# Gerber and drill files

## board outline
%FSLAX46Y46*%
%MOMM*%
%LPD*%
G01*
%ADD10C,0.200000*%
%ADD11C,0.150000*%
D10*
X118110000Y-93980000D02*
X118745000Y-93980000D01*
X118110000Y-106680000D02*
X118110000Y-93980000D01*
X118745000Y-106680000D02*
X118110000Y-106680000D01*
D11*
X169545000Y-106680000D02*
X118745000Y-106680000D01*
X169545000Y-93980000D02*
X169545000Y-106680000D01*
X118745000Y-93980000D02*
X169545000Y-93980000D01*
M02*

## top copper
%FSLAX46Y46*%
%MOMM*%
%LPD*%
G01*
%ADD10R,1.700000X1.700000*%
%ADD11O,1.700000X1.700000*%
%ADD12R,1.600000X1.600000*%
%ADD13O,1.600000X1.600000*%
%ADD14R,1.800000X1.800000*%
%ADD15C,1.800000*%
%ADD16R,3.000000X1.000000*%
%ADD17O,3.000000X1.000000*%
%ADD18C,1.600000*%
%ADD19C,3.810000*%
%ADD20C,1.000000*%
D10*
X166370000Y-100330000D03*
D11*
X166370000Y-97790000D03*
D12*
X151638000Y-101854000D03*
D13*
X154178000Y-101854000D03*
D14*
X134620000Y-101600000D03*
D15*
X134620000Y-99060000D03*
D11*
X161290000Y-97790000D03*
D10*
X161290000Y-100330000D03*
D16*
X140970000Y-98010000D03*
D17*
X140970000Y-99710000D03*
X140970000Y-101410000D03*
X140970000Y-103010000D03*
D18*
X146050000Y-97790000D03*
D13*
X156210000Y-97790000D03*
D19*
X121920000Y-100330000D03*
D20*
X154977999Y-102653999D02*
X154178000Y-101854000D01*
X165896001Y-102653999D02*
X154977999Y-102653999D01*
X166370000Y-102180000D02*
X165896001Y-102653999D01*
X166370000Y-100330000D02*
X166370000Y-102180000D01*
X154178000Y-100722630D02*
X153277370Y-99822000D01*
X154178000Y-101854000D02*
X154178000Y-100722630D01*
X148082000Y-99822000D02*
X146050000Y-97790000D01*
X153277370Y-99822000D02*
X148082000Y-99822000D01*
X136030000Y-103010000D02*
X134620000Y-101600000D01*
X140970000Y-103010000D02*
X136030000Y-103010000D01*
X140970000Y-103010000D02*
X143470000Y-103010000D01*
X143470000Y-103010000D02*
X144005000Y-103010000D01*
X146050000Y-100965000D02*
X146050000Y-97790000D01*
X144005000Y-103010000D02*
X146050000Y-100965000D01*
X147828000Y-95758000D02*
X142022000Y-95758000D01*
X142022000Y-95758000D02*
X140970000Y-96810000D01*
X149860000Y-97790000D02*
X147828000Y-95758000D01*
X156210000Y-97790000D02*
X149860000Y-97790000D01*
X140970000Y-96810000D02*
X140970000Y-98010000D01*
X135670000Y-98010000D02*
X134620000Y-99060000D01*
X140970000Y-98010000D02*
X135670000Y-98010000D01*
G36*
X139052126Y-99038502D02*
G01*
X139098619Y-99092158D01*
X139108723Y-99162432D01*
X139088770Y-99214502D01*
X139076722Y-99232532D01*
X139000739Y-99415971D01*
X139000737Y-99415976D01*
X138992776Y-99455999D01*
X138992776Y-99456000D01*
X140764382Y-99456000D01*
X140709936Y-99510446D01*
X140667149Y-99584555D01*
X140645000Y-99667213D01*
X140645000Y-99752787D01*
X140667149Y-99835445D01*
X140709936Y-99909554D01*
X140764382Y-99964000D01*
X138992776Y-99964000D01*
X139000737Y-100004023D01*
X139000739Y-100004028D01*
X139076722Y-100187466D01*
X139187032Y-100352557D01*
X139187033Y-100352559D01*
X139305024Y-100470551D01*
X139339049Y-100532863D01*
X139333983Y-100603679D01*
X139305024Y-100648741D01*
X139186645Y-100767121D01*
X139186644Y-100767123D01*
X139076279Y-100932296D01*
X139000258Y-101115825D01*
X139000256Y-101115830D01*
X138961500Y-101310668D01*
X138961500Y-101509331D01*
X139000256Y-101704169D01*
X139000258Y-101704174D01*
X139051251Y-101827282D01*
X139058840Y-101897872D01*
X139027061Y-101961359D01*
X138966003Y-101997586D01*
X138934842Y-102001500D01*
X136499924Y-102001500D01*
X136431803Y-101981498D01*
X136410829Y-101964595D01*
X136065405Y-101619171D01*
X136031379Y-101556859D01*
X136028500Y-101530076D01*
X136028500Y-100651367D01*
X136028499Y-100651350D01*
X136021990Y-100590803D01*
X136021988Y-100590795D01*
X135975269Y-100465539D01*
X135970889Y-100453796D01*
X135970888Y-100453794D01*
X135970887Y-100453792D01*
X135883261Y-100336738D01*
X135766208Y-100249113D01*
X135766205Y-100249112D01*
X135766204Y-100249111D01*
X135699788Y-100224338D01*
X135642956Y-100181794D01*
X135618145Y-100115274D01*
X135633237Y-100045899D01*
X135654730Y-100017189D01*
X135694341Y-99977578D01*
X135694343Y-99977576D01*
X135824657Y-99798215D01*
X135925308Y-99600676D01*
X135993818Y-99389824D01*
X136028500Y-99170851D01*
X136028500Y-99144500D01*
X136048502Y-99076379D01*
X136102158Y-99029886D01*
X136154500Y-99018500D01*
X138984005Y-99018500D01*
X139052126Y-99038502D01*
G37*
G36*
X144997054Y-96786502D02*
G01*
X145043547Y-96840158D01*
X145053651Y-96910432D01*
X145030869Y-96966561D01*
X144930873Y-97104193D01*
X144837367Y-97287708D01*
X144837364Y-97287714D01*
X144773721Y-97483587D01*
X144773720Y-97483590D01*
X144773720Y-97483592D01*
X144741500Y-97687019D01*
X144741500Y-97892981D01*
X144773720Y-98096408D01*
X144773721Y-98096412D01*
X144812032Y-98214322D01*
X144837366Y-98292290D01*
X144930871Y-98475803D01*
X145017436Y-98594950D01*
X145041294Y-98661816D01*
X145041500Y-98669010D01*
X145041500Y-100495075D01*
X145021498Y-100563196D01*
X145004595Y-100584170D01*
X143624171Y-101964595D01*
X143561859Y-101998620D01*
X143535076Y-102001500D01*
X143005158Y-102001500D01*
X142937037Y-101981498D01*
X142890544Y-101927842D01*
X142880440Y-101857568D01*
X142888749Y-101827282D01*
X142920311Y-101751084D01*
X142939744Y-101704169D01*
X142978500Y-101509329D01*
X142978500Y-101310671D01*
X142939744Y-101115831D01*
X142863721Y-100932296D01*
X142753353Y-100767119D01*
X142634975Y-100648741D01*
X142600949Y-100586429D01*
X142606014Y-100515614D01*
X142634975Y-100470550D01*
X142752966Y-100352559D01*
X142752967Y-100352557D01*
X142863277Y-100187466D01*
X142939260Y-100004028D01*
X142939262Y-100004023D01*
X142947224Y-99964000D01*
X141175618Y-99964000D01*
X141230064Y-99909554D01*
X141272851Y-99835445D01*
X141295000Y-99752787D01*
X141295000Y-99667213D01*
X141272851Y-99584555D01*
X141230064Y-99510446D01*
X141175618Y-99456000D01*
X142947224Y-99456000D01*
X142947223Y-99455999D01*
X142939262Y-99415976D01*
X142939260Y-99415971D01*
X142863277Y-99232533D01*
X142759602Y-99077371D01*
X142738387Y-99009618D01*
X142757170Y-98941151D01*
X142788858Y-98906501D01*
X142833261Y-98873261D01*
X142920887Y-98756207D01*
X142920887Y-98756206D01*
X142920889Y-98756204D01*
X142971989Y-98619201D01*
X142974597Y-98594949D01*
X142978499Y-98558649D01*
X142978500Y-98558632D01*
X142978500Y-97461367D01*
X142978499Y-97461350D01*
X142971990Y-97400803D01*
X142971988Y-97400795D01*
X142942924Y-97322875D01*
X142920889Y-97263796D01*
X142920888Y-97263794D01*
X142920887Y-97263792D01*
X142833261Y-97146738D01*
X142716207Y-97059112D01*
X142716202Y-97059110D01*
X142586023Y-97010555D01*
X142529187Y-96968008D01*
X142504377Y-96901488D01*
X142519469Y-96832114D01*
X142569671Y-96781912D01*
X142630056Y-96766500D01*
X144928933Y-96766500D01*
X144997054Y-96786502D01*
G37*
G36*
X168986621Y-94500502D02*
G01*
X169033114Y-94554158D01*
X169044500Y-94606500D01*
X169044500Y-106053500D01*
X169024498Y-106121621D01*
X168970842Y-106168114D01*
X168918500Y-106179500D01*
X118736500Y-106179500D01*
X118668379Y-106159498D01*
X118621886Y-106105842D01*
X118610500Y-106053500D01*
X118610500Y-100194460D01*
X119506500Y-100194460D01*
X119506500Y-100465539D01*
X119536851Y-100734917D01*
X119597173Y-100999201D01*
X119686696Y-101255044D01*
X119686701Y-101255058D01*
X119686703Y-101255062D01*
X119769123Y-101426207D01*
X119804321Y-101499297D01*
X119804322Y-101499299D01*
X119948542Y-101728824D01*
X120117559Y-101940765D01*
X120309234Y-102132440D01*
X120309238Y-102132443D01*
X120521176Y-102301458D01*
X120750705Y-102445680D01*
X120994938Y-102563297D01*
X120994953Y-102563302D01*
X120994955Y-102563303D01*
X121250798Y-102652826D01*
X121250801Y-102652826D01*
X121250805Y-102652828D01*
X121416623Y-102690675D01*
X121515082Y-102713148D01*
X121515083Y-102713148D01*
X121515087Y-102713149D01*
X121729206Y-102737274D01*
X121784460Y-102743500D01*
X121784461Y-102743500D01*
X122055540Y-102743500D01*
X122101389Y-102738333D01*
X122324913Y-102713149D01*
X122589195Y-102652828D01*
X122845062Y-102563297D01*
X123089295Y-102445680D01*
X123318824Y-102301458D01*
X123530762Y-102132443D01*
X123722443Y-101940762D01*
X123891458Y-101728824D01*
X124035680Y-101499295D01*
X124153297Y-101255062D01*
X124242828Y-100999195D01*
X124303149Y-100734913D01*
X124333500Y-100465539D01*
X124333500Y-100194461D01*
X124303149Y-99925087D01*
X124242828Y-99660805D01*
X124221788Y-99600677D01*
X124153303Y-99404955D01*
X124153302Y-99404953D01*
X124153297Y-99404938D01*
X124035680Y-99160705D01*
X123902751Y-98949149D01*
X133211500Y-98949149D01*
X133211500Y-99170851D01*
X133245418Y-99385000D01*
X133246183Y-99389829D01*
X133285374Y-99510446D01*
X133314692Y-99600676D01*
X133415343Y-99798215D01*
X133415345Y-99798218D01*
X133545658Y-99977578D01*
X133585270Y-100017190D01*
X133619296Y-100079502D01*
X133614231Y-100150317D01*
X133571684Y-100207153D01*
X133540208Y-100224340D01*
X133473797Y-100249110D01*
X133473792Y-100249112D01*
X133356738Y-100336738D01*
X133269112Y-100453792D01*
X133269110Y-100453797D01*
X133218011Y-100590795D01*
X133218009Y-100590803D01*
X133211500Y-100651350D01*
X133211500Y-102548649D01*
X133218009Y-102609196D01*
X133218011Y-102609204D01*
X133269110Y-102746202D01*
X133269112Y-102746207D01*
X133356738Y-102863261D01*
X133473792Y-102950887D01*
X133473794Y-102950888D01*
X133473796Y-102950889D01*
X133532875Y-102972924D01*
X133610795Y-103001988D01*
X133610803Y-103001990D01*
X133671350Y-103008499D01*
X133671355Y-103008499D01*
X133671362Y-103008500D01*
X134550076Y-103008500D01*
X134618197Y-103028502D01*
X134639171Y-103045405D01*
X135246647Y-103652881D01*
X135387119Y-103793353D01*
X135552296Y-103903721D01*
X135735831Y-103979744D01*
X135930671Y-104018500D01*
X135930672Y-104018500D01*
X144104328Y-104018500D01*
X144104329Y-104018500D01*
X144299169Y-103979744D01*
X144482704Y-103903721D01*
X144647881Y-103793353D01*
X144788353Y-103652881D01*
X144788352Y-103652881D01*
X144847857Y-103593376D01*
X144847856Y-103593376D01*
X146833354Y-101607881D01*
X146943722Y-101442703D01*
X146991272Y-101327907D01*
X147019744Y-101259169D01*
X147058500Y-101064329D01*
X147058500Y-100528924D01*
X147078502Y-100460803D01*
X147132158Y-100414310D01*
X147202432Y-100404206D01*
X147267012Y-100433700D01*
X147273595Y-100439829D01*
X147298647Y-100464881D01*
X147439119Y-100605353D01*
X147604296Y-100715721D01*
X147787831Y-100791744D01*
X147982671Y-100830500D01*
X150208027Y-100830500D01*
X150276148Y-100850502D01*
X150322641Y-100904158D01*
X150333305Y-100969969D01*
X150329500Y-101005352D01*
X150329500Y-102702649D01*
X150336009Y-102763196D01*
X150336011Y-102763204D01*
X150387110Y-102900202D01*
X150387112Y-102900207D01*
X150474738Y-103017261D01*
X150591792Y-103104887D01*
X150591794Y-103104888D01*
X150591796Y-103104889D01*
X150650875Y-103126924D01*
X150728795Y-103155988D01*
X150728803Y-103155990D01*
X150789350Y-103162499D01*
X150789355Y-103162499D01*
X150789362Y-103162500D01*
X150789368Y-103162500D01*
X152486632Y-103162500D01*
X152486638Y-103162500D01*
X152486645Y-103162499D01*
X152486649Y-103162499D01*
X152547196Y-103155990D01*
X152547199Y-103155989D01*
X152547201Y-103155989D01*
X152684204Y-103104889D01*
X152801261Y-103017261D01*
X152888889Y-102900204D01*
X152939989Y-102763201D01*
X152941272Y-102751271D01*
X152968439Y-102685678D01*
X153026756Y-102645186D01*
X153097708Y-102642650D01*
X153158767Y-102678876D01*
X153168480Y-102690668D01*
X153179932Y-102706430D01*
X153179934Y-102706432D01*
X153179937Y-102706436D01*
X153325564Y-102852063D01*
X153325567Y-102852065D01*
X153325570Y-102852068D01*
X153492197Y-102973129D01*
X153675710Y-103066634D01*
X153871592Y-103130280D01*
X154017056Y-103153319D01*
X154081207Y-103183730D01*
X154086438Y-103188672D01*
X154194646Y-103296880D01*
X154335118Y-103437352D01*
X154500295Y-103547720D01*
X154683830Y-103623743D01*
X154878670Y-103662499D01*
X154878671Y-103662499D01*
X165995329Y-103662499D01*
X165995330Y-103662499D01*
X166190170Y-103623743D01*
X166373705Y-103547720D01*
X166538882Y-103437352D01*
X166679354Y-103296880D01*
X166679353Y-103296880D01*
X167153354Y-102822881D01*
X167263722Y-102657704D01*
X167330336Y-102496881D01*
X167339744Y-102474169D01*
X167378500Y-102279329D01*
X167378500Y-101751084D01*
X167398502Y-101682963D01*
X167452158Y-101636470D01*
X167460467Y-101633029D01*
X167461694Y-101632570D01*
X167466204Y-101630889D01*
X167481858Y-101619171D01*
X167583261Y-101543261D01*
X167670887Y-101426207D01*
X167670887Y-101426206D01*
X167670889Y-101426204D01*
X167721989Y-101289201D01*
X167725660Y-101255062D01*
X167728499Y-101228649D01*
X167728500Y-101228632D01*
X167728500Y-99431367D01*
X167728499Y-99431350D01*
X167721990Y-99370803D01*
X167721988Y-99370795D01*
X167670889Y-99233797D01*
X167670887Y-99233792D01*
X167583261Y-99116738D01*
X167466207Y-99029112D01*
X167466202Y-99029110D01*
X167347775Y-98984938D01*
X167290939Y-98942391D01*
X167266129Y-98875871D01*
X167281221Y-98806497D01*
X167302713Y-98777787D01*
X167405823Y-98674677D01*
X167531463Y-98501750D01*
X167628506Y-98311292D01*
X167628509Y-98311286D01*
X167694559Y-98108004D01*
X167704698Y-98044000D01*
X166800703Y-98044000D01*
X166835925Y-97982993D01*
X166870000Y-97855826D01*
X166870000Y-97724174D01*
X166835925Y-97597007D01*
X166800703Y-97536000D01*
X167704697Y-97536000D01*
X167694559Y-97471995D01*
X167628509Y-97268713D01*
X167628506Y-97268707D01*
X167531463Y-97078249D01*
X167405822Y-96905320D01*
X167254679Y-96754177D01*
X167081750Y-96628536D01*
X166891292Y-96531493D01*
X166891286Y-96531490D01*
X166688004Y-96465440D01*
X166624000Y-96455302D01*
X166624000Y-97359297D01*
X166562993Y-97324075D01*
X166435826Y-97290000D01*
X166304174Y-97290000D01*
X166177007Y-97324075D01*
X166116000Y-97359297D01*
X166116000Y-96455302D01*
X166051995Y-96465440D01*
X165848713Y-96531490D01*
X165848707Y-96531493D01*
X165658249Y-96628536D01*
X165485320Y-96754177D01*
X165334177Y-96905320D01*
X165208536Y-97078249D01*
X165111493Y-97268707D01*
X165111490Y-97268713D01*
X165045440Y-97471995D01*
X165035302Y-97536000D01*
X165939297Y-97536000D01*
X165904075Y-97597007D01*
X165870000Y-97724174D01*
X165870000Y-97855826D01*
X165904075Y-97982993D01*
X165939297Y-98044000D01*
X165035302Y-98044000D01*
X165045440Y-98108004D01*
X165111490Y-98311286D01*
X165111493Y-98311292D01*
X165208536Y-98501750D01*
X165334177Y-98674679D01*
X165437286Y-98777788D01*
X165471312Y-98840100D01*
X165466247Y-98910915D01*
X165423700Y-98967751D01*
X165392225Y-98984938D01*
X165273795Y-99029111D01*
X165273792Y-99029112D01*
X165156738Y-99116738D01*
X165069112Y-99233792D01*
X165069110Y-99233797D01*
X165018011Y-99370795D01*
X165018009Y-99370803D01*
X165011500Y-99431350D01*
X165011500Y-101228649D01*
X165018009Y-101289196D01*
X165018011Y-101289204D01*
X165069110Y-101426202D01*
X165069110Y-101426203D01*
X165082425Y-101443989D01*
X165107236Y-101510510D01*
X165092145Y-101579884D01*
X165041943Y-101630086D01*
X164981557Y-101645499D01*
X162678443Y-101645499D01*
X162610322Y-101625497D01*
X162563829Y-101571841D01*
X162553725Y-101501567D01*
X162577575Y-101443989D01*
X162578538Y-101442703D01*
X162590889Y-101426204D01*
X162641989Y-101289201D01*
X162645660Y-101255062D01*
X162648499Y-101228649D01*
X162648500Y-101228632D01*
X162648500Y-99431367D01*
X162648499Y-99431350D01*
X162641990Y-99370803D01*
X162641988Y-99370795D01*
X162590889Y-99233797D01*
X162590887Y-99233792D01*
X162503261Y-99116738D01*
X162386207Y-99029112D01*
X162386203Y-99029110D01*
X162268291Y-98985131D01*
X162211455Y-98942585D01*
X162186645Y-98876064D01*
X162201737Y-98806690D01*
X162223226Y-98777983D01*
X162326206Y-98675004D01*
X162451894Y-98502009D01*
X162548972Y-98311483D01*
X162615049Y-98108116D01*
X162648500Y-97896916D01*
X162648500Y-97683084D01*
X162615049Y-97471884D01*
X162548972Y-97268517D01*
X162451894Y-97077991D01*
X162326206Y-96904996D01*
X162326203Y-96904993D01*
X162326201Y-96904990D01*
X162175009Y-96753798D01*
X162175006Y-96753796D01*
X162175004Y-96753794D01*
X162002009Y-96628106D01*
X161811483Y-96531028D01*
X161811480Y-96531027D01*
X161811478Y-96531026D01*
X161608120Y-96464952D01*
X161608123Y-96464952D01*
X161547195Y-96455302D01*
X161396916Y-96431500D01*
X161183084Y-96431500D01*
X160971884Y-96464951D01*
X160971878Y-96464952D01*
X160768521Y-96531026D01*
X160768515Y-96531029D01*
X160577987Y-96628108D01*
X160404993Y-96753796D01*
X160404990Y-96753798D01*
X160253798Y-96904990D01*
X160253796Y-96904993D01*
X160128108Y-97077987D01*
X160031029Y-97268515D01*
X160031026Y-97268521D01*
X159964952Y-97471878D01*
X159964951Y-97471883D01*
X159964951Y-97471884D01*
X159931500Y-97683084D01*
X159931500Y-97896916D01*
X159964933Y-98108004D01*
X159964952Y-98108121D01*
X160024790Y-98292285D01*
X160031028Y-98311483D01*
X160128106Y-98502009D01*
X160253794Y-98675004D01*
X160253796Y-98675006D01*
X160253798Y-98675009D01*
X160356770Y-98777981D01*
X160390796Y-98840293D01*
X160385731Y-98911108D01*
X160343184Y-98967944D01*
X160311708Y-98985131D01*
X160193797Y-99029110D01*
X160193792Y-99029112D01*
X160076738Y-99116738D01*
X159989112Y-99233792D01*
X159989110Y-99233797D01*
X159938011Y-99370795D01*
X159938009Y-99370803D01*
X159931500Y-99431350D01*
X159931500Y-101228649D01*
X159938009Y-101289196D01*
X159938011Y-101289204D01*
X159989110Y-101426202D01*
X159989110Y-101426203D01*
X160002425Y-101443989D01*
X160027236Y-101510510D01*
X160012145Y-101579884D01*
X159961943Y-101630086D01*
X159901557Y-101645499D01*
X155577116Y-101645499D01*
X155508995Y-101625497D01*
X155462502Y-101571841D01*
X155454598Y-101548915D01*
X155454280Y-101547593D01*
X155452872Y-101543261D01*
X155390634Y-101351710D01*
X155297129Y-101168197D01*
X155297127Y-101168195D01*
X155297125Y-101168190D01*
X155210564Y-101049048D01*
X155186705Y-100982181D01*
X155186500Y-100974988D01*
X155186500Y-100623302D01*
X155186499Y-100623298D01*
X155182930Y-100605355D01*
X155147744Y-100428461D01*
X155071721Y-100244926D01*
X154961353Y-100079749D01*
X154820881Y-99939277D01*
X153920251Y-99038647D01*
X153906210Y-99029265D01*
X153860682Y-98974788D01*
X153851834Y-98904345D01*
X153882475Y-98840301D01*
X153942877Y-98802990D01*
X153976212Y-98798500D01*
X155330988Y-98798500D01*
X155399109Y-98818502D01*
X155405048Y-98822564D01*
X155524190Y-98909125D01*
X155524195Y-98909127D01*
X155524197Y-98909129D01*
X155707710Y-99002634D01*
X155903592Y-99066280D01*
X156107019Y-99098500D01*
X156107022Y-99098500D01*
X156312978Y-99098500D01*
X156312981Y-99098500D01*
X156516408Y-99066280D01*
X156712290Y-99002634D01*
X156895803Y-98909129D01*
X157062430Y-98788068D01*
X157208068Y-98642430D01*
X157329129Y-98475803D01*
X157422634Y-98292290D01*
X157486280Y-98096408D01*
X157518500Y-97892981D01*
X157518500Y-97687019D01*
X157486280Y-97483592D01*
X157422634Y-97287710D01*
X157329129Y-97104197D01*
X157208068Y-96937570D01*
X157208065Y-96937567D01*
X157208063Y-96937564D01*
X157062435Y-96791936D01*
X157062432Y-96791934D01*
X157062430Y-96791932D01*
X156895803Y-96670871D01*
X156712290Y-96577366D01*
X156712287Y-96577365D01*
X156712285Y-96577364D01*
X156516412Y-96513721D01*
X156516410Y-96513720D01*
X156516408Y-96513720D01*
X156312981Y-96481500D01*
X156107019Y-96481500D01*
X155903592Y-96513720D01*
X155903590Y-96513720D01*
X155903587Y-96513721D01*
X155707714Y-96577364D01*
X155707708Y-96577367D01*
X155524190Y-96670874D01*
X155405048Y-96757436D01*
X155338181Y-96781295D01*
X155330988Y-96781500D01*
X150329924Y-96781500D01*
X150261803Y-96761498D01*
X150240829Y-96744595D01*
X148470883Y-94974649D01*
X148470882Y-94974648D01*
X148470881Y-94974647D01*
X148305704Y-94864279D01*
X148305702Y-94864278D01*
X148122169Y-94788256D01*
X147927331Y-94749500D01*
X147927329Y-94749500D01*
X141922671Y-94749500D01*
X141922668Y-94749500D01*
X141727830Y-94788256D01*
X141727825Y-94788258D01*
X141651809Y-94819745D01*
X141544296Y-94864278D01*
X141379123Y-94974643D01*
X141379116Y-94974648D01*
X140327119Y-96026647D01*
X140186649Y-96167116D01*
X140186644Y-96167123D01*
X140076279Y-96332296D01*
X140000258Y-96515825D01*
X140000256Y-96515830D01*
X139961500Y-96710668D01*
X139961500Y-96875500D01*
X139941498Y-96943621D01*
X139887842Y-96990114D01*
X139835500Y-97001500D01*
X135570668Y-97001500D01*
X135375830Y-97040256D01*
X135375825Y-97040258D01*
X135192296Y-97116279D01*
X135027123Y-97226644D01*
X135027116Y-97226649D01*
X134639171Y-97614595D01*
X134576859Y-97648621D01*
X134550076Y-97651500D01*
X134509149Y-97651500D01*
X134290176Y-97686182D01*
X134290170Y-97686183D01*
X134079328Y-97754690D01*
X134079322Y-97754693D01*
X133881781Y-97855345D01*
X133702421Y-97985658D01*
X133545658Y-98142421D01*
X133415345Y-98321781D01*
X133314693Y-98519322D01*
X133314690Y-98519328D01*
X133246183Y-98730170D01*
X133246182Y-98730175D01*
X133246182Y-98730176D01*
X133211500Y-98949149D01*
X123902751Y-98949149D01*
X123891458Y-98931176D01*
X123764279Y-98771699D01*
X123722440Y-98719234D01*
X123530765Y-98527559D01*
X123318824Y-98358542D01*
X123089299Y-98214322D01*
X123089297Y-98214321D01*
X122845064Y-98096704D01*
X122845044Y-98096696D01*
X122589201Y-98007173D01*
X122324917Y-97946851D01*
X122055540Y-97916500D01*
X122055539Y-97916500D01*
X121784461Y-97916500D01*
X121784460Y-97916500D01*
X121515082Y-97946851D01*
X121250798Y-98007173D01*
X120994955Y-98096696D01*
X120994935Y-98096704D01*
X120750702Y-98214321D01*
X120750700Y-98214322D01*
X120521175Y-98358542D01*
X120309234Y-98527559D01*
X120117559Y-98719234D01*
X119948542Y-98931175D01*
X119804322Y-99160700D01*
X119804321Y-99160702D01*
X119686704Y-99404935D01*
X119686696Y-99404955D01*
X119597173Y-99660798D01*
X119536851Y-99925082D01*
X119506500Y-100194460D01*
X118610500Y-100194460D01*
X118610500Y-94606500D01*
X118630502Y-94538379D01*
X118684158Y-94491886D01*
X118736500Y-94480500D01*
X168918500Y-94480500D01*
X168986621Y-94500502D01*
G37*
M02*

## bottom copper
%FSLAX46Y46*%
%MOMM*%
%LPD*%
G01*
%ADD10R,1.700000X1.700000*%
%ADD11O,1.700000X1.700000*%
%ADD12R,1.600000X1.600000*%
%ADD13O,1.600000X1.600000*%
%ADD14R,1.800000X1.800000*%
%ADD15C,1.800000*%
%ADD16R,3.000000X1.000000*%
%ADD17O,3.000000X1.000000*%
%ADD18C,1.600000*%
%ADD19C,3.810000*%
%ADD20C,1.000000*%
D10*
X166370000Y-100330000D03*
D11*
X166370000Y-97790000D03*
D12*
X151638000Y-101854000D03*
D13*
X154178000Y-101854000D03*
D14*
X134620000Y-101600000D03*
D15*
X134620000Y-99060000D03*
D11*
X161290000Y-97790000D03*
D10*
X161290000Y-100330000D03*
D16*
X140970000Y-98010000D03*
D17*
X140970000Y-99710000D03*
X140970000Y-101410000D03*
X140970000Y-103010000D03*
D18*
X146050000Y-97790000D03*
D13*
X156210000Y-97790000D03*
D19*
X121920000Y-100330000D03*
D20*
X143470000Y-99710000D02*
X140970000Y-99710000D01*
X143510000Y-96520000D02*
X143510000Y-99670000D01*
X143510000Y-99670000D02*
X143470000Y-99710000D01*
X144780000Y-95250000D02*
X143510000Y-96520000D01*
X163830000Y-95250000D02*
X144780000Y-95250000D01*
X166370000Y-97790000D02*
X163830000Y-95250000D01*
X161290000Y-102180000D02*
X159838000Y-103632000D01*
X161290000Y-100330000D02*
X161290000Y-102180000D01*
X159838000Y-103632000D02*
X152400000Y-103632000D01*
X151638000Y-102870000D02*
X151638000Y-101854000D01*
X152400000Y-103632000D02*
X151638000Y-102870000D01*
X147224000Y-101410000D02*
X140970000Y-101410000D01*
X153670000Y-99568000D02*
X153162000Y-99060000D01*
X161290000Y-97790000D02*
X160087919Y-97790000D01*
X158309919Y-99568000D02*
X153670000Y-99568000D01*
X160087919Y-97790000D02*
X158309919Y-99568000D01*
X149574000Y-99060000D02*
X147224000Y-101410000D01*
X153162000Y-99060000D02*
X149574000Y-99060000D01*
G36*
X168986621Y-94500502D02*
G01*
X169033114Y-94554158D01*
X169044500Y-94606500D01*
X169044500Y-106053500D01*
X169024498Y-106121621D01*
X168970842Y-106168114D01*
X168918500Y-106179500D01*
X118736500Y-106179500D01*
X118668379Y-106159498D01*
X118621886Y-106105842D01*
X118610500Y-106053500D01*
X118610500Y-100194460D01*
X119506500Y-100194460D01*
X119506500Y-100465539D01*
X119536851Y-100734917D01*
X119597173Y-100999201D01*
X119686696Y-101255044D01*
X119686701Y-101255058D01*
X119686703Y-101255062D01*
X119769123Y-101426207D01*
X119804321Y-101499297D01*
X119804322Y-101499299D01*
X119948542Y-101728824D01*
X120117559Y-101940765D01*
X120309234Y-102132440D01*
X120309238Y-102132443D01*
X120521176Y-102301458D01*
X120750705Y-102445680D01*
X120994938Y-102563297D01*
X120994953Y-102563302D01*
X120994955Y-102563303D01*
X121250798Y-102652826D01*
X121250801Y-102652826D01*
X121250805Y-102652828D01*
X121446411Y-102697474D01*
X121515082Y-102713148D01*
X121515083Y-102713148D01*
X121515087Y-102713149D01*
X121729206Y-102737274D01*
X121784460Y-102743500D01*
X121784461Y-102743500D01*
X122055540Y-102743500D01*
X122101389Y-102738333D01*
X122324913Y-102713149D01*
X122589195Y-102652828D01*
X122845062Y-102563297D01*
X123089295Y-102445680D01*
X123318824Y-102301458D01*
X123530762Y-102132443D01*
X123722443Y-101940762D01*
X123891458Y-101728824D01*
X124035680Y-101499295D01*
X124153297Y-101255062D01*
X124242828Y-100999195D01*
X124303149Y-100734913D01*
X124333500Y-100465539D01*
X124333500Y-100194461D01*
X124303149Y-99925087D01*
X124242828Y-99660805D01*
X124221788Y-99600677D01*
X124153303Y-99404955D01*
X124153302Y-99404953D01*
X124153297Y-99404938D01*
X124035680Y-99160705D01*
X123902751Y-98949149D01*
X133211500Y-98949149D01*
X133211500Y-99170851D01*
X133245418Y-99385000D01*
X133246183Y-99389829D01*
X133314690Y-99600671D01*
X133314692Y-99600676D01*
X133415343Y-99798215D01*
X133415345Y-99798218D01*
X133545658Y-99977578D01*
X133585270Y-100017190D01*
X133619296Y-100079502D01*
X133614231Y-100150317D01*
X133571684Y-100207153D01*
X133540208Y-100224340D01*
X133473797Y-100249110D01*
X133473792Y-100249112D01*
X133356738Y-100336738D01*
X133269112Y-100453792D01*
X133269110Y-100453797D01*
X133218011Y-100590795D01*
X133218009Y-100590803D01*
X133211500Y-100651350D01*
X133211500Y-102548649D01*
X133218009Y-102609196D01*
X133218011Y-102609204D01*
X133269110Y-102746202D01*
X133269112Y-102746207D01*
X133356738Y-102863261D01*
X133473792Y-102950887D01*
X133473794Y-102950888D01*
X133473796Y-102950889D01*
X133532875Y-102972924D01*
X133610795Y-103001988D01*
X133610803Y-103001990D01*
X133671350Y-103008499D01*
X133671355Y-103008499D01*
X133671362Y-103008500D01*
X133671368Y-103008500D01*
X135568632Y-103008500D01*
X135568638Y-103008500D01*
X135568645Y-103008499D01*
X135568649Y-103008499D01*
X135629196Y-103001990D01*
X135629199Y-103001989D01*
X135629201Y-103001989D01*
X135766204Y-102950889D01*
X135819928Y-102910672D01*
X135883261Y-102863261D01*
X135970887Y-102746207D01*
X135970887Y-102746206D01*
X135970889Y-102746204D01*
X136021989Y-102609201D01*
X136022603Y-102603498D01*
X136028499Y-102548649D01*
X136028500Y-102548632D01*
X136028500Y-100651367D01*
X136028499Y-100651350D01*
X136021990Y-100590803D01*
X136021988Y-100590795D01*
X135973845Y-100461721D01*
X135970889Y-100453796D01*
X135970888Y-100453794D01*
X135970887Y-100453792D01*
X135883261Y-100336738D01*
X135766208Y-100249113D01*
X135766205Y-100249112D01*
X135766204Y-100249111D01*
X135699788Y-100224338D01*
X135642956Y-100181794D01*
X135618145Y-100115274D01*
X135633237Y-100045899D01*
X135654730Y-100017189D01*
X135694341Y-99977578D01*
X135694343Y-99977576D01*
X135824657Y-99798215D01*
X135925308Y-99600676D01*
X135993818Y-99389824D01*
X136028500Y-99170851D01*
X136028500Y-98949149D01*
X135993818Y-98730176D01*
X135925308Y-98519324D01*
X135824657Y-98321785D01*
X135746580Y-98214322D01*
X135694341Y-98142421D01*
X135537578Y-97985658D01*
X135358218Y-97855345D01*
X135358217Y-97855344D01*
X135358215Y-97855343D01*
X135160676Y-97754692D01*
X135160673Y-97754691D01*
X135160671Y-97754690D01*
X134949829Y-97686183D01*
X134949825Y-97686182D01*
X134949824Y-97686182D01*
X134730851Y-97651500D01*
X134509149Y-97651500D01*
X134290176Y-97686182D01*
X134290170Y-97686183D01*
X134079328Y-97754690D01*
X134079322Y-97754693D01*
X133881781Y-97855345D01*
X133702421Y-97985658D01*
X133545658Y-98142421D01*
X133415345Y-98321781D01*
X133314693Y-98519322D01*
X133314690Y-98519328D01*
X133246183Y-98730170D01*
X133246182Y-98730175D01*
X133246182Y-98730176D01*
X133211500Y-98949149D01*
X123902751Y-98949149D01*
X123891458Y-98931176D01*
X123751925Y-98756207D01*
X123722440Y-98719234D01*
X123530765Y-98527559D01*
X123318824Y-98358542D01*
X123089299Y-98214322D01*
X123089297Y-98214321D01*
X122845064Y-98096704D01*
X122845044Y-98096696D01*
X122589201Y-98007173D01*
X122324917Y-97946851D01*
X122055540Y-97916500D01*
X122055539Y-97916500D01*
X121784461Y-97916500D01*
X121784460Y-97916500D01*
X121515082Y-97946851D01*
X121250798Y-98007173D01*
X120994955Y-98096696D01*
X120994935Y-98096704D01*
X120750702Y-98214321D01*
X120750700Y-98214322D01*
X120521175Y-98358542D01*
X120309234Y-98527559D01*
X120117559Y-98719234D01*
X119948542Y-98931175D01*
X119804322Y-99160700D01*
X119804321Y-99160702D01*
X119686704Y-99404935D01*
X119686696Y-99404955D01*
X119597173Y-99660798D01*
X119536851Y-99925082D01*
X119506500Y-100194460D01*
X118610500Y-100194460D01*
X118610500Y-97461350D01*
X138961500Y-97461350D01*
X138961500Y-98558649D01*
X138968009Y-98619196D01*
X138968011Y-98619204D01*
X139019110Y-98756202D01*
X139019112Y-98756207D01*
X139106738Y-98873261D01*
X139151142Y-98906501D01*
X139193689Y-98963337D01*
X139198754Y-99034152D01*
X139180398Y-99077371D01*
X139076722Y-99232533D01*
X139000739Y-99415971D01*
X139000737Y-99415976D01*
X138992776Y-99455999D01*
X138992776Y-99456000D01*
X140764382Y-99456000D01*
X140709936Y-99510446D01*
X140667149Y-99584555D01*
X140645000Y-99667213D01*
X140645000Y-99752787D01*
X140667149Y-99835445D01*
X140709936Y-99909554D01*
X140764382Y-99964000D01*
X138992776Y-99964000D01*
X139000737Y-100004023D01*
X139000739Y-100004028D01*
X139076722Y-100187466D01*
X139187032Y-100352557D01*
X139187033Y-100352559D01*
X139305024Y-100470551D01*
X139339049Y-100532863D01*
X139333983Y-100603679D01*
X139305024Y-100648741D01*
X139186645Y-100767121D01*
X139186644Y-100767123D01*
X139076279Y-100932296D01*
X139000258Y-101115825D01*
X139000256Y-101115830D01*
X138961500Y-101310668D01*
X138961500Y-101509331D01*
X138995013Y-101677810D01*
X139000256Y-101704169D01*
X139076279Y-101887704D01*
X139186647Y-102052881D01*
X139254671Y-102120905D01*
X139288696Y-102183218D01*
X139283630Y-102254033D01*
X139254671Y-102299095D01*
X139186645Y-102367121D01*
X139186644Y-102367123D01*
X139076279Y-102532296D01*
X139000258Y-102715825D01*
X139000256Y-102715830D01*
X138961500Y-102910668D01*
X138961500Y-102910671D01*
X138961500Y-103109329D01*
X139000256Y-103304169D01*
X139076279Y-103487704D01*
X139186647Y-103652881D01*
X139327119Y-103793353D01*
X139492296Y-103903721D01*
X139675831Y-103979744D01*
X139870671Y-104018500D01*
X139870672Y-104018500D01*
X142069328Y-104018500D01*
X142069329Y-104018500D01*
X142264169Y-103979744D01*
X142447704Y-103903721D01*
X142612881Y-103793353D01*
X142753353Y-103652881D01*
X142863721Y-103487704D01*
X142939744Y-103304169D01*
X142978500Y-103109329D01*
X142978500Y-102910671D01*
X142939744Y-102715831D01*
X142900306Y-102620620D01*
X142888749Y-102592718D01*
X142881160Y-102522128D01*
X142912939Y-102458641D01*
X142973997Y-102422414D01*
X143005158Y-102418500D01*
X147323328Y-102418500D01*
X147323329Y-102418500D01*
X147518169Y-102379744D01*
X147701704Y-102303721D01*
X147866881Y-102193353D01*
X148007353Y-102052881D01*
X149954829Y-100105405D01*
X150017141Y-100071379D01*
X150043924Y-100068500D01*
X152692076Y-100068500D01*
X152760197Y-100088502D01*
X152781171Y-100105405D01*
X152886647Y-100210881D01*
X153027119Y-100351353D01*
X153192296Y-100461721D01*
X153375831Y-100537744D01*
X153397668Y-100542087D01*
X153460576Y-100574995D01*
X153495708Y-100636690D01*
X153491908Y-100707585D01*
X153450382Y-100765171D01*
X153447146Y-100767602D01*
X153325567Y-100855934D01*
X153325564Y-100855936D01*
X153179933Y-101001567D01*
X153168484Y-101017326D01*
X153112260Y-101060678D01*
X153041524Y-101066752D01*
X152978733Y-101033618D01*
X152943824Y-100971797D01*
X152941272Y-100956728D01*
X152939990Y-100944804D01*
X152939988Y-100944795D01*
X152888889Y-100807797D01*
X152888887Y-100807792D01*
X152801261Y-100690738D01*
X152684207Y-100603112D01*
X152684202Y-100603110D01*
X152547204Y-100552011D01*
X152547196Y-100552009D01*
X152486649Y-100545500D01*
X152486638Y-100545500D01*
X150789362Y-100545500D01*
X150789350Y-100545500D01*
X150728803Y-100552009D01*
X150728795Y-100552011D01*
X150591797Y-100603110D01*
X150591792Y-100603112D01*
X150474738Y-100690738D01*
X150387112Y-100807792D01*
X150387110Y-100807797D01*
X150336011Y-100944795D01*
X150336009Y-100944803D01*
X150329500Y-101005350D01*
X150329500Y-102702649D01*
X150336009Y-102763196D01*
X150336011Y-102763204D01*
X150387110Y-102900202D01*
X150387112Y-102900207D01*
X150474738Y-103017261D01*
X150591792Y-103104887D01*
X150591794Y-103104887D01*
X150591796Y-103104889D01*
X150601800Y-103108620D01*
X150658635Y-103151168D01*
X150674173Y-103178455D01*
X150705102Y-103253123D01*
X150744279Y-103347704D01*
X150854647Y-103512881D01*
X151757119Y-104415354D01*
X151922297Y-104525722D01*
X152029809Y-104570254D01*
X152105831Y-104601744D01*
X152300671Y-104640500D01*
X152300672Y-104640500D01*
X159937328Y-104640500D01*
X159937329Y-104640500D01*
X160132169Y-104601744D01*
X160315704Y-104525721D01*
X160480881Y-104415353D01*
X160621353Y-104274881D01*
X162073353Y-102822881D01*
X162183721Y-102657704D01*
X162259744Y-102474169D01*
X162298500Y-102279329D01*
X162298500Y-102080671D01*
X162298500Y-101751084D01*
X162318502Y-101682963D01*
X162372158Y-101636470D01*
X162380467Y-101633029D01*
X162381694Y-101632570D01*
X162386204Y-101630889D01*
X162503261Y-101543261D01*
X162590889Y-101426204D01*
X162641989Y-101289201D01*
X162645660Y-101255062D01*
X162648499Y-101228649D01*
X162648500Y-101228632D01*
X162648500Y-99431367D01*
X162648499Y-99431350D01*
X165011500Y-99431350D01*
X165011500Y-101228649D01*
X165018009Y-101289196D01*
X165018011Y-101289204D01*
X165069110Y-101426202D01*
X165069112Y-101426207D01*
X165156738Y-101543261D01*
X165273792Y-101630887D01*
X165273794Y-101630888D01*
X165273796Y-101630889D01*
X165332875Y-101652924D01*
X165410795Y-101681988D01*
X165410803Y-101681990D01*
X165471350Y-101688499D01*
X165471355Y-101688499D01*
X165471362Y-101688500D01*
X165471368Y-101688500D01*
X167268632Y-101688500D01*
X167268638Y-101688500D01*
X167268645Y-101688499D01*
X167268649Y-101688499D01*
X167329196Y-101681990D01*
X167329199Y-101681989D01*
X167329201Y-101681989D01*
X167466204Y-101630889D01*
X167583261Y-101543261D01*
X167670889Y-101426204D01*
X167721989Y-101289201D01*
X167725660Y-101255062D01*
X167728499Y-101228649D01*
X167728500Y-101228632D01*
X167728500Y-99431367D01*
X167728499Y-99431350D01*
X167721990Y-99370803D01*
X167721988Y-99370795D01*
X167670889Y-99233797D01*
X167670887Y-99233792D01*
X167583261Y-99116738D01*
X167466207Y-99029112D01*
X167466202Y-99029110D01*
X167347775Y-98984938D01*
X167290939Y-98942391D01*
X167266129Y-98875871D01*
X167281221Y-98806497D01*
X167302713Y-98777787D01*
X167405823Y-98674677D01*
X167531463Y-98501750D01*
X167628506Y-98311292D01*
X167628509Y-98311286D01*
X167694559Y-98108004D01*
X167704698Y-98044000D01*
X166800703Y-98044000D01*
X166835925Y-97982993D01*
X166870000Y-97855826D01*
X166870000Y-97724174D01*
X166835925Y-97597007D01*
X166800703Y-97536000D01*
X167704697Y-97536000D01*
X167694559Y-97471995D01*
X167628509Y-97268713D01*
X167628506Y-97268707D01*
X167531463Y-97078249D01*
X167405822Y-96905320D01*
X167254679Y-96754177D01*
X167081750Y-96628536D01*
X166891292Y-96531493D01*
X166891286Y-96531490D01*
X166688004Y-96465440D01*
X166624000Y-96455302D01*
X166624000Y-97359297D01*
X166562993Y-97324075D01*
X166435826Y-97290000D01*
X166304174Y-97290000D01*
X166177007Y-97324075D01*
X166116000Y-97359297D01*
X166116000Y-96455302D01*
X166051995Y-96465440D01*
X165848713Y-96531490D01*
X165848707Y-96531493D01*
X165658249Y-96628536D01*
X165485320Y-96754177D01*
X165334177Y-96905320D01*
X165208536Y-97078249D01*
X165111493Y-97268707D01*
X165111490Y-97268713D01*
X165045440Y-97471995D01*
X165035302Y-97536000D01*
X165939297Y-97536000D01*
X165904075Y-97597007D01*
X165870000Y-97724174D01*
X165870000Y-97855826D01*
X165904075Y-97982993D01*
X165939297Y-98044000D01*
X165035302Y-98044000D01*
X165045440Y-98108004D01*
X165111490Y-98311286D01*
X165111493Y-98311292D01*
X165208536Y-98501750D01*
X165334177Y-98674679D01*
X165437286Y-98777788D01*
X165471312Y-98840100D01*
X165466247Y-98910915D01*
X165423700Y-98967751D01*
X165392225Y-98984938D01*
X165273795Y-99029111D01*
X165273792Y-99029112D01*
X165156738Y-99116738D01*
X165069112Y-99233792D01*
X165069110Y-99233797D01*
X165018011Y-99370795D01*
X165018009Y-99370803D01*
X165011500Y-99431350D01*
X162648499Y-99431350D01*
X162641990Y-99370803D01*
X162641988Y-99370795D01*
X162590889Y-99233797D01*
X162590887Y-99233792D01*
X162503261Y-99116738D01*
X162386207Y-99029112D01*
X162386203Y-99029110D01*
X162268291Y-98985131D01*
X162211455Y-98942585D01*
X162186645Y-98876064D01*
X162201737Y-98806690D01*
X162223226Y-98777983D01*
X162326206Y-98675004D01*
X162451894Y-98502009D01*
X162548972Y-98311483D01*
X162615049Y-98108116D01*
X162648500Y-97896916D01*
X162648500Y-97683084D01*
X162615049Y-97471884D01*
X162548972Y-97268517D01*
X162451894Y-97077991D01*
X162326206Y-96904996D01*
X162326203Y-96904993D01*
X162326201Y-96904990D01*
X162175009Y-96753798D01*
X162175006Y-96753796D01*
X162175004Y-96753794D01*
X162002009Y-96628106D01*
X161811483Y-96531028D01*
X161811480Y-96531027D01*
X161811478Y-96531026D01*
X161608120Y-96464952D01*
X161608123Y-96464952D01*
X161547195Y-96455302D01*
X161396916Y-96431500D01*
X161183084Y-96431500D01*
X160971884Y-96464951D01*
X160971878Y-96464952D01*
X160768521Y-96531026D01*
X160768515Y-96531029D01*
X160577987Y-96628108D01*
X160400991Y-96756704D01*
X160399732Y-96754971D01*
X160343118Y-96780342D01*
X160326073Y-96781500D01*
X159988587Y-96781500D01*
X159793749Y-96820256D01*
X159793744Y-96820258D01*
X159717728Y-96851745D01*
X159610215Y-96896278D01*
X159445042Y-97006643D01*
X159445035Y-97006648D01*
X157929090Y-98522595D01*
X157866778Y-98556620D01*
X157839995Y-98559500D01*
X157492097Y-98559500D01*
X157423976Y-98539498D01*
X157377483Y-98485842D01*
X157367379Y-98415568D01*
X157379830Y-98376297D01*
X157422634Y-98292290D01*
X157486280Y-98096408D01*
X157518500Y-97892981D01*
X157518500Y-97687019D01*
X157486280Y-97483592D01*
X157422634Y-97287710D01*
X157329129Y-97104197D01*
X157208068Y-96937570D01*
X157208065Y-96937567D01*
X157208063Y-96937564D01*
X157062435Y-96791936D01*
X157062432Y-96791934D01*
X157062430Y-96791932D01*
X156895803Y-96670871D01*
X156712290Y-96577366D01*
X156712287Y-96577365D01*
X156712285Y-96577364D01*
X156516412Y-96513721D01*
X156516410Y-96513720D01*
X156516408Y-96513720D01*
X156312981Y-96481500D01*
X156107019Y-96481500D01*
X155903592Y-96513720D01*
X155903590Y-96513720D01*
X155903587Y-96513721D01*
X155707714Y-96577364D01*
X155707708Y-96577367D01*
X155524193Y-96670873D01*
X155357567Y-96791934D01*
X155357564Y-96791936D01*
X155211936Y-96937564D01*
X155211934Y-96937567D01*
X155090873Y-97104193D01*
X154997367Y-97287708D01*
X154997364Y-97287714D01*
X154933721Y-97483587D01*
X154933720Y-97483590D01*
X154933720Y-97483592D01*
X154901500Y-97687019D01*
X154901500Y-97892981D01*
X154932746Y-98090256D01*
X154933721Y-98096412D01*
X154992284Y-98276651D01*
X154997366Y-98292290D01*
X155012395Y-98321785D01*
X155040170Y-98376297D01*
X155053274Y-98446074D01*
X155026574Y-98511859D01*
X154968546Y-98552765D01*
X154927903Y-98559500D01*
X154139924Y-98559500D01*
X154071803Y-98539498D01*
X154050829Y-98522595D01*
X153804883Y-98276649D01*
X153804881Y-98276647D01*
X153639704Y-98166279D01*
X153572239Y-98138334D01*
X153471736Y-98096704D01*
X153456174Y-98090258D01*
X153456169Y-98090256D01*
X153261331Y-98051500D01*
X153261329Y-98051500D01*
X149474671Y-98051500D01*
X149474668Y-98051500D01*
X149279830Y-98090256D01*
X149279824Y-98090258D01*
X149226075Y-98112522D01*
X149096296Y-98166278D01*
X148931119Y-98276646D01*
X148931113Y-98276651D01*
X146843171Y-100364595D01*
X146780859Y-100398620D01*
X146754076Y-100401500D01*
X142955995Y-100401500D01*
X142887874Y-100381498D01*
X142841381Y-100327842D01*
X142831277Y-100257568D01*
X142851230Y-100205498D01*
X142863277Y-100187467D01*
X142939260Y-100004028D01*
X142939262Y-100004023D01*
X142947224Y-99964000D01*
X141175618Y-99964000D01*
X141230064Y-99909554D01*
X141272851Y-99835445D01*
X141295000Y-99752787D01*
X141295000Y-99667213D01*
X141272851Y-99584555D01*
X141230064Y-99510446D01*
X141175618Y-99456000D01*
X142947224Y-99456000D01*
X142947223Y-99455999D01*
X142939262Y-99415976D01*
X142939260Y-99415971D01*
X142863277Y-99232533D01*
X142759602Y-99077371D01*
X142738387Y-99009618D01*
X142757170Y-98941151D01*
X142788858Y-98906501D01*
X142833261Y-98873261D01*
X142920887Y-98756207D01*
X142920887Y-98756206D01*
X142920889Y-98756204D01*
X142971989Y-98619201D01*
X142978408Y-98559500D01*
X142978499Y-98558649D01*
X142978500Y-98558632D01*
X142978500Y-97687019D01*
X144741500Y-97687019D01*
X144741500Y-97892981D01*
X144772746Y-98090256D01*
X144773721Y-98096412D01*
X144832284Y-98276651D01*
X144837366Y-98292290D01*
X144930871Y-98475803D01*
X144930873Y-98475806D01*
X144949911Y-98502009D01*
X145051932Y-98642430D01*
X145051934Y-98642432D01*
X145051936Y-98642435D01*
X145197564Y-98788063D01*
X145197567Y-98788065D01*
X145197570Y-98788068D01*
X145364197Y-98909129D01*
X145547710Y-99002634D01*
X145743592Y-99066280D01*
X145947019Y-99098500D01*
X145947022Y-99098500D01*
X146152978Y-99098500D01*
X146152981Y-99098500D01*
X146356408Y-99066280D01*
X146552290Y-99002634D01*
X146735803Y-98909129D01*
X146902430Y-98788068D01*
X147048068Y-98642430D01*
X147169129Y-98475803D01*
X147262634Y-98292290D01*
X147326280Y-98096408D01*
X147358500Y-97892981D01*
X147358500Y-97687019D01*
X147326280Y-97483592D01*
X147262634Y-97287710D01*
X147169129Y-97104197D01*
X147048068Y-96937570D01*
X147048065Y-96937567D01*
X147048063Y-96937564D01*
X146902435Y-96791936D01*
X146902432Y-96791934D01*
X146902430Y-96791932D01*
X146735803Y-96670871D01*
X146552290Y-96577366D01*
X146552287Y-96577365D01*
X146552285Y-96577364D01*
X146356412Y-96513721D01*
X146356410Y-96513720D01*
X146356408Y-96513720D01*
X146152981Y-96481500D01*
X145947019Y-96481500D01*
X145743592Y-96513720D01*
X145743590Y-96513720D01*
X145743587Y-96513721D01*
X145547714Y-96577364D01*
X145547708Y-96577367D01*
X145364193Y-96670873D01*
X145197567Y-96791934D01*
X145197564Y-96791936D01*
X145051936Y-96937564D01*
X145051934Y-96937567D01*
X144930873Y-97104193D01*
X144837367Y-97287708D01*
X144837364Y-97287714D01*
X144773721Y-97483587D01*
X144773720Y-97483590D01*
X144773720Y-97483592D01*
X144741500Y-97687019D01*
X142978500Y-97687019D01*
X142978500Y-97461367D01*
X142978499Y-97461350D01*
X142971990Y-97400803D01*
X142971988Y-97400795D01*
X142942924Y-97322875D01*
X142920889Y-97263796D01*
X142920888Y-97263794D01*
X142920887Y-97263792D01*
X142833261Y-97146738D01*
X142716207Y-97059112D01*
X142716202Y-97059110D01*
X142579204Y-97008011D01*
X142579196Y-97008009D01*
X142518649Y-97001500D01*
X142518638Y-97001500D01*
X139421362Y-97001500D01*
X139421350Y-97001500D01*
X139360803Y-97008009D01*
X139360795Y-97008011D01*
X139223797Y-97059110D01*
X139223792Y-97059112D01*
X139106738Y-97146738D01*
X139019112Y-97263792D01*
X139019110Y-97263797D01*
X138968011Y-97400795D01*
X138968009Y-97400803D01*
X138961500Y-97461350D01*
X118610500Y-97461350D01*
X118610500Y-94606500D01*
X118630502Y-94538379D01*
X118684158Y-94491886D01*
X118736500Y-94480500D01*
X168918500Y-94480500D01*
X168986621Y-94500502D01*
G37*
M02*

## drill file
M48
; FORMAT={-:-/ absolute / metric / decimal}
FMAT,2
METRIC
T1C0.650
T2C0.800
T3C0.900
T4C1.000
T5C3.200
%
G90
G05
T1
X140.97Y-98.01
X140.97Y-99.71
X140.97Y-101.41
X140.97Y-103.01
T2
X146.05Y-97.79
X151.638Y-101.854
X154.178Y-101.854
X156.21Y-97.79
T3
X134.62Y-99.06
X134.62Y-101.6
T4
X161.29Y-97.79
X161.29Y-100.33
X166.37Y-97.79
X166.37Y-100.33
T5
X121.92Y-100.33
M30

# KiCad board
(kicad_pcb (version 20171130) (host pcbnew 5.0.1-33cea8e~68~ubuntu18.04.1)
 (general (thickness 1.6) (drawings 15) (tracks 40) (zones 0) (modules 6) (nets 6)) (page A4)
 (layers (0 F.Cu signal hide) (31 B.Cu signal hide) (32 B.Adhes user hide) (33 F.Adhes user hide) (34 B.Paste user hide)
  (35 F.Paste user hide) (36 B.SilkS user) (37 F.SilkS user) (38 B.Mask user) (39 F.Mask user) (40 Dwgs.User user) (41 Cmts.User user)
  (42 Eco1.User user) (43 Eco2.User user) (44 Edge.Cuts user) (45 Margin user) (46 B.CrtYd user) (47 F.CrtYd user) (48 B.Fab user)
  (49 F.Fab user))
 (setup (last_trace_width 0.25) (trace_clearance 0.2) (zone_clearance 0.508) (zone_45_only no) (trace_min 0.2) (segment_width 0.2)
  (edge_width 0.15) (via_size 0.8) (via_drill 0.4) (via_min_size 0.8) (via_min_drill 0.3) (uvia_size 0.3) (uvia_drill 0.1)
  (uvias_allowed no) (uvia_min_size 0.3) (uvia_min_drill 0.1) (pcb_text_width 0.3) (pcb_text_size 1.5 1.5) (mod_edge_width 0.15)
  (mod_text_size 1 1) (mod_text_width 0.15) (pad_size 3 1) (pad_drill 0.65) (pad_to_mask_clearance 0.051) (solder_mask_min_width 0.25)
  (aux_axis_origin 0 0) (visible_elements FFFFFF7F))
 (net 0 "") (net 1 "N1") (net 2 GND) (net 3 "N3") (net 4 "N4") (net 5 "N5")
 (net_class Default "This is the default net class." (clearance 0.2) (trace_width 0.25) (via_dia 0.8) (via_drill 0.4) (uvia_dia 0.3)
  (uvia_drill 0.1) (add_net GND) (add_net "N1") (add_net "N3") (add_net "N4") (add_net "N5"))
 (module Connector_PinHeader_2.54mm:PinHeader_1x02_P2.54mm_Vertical (layer F.Cu) (at 166.37 100.33 180)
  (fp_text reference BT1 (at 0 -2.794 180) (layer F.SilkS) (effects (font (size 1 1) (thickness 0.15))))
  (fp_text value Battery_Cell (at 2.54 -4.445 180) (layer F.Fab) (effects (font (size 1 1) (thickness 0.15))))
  (pad 1 thru_hole rect (at 0 0 180) (size 1.7 1.7) (drill 1) (layers *.Cu *.Mask) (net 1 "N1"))
  (pad 2 thru_hole oval (at 0 2.54 180) (size 1.7 1.7) (drill 1) (layers *.Cu *.Mask) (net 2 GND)))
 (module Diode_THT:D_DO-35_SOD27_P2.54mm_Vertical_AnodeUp (layer F.Cu) (at 151.638 101.854)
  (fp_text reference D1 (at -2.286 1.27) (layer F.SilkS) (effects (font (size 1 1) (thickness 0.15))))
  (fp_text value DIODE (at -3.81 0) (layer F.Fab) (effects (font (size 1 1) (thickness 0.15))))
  (pad 1 thru_hole rect (at 0 0) (size 1.6 1.6) (drill 0.8) (layers *.Cu *.Mask) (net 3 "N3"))
  (pad 2 thru_hole oval (at 2.54 0) (size 1.6 1.6) (drill 0.8) (layers *.Cu *.Mask) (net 1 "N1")))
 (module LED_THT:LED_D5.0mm (layer B.Cu) (at 134.62 101.6 90)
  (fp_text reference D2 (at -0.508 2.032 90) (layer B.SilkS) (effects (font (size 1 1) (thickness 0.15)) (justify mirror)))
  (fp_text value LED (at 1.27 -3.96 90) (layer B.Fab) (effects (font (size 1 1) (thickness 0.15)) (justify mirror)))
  (pad 1 thru_hole rect (at 0 0 90) (size 1.8 1.8) (drill 0.9) (layers *.Cu *.Mask) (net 1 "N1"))
  (pad 2 thru_hole circle (at 2.54 0 90) (size 1.8 1.8) (drill 0.9) (layers *.Cu *.Mask) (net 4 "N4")))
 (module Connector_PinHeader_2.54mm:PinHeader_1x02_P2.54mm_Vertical (layer F.Cu) (at 161.29 100.33 180)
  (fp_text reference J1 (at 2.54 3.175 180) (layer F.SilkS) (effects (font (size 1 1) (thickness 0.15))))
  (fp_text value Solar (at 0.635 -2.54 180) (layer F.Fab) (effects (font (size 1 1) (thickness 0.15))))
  (pad 2 thru_hole oval (at 0 2.54 180) (size 1.7 1.7) (drill 1) (layers *.Cu *.Mask) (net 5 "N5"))
  (pad 1 thru_hole rect (at 0 0 180) (size 1.7 1.7) (drill 1) (layers *.Cu *.Mask) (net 3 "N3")))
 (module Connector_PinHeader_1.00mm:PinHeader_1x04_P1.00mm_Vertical (layer F.Cu) (at 140.97 99.06)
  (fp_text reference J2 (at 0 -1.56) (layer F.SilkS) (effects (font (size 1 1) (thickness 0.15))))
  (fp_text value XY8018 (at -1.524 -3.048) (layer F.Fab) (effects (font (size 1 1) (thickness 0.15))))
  (pad 1 thru_hole rect (at 0 -1.05) (size 3 1) (drill 0.65) (layers *.Cu *.Mask) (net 4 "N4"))
  (pad 2 thru_hole oval (at 0 0.65) (size 3 1) (drill 0.65) (layers *.Cu *.Mask) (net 2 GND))
  (pad 3 thru_hole oval (at 0 2.35) (size 3 1) (drill 0.65) (layers *.Cu *.Mask) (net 5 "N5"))
  (pad 4 thru_hole oval (at 0 3.95) (size 3 1) (drill 0.65) (layers *.Cu *.Mask) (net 1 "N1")))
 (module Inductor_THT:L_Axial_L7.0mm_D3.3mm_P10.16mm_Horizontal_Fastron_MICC (layer F.Cu) (at 146.05 97.79)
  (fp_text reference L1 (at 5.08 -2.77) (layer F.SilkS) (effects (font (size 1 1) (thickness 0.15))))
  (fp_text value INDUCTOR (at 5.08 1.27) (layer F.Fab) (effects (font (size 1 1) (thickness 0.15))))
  (pad 1 thru_hole circle (at 0 0) (size 1.6 1.6) (drill 0.8) (layers *.Cu *.Mask) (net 1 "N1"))
  (pad 2 thru_hole oval (at 10.16 0) (size 1.6 1.6) (drill 0.8) (layers *.Cu *.Mask) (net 4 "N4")))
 (gr_line (start 118.11 93.98) (end 118.745 93.98) (layer Edge.Cuts) (width 0.2))
 (gr_line (start 118.11 106.68) (end 118.11 93.98) (layer Edge.Cuts) (width 0.2))
 (gr_line (start 118.745 106.68) (end 118.11 106.68) (layer Edge.Cuts) (width 0.2))
 (gr_line (start 169.545 106.68) (end 118.745 106.68) (layer Edge.Cuts) (width 0.15))
 (gr_line (start 169.545 93.98) (end 169.545 106.68) (layer Edge.Cuts) (width 0.15))
 (gr_line (start 118.745 93.98) (end 169.545 93.98) (layer Edge.Cuts) (width 0.15))
 (via (at 121.92 100.33) (size 3.81) (drill 3.2004) (layers F.Cu B.Cu) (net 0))
 (segment (start 154.977999 102.653999) (end 154.178 101.854) (width 1) (layer F.Cu) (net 1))
 (segment (start 165.896001 102.653999) (end 154.977999 102.653999) (width 1) (layer F.Cu) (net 1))
 (segment (start 166.37 102.18) (end 165.896001 102.653999) (width 1) (layer F.Cu) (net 1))
 (segment (start 166.37 100.33) (end 166.37 102.18) (width 1) (layer F.Cu) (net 1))
 (segment (start 154.178 100.72263) (end 153.27737 99.822) (width 1) (layer F.Cu) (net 1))
 (segment (start 154.178 101.854) (end 154.178 100.72263) (width 1) (layer F.Cu) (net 1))
 (segment (start 148.082 99.822) (end 146.05 97.79) (width 1) (layer F.Cu) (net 1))
 (segment (start 153.27737 99.822) (end 148.082 99.822) (width 1) (layer F.Cu) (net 1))
 (segment (start 136.03 103.01) (end 134.62 101.6) (width 1) (layer F.Cu) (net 1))
 (segment (start 140.97 103.01) (end 136.03 103.01) (width 1) (layer F.Cu) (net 1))
 (segment (start 140.97 103.01) (end 143.47 103.01) (width 1) (layer F.Cu) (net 1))
 (segment (start 143.47 103.01) (end 144.005 103.01) (width 1) (layer F.Cu) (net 1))
 (segment (start 146.05 100.965) (end 146.05 97.79) (width 1) (layer F.Cu) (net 1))
 (segment (start 144.005 103.01) (end 146.05 100.965) (width 1) (layer F.Cu) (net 1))
 (segment (start 143.47 99.71) (end 140.97 99.71) (width 1) (layer B.Cu) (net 2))
 (segment (start 143.51 96.52) (end 143.51 99.67) (width 1) (layer B.Cu) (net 2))
 (segment (start 143.51 99.67) (end 143.47 99.71) (width 1) (layer B.Cu) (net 2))
 (segment (start 144.78 95.25) (end 143.51 96.52) (width 1) (layer B.Cu) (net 2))
 (segment (start 163.83 95.25) (end 144.78 95.25) (width 1) (layer B.Cu) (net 2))
 (segment (start 166.37 97.79) (end 163.83 95.25) (width 1) (layer B.Cu) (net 2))
 (segment (start 161.29 102.18) (end 159.838 103.632) (width 1) (layer B.Cu) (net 3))
 (segment (start 161.29 100.33) (end 161.29 102.18) (width 1) (layer B.Cu) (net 3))
 (segment (start 159.838 103.632) (end 152.4 103.632) (width 1) (layer B.Cu) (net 3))
 (segment (start 151.638 102.87) (end 151.638 101.854) (width 1) (layer B.Cu) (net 3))
 (segment (start 152.4 103.632) (end 151.638 102.87) (width 1) (layer B.Cu) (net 3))
 (segment (start 147.828 95.758) (end 142.022 95.758) (width 1) (layer F.Cu) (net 4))
 (segment (start 142.022 95.758) (end 140.97 96.81) (width 1) (layer F.Cu) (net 4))
 (segment (start 149.86 97.79) (end 147.828 95.758) (width 1) (layer F.Cu) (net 4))
 (segment (start 156.21 97.79) (end 149.86 97.79) (width 1) (layer F.Cu) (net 4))
 (segment (start 140.97 96.81) (end 140.97 98.01) (width 1) (layer F.Cu) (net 4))
 (segment (start 135.67 98.01) (end 134.62 99.06) (width 1) (layer F.Cu) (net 4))
 (segment (start 140.97 98.01) (end 135.67 98.01) (width 1) (layer F.Cu) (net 4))
 (segment (start 147.224 101.41) (end 140.97 101.41) (width 1) (layer B.Cu) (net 5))
 (segment (start 153.67 99.568) (end 153.162 99.06) (width 1) (layer B.Cu) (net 5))
 (segment (start 161.29 97.79) (end 160.087919 97.79) (width 1) (layer B.Cu) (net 5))
 (segment (start 158.309919 99.568) (end 153.67 99.568) (width 1) (layer B.Cu) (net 5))
 (segment (start 160.087919 97.79) (end 158.309919 99.568) (width 1) (layer B.Cu) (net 5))
 (segment (start 149.574 99.06) (end 147.224 101.41) (width 1) (layer B.Cu) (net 5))
 (segment (start 153.162 99.06) (end 149.574 99.06) (width 1) (layer B.Cu) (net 5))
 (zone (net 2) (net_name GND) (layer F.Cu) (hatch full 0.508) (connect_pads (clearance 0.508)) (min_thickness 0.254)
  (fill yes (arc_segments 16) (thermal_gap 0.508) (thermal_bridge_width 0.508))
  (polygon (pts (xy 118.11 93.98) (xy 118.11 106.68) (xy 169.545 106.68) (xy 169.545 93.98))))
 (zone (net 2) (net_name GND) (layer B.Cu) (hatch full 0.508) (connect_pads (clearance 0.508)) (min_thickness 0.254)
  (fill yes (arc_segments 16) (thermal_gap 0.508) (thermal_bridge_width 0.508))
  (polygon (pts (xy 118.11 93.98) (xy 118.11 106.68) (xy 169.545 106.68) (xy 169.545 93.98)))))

